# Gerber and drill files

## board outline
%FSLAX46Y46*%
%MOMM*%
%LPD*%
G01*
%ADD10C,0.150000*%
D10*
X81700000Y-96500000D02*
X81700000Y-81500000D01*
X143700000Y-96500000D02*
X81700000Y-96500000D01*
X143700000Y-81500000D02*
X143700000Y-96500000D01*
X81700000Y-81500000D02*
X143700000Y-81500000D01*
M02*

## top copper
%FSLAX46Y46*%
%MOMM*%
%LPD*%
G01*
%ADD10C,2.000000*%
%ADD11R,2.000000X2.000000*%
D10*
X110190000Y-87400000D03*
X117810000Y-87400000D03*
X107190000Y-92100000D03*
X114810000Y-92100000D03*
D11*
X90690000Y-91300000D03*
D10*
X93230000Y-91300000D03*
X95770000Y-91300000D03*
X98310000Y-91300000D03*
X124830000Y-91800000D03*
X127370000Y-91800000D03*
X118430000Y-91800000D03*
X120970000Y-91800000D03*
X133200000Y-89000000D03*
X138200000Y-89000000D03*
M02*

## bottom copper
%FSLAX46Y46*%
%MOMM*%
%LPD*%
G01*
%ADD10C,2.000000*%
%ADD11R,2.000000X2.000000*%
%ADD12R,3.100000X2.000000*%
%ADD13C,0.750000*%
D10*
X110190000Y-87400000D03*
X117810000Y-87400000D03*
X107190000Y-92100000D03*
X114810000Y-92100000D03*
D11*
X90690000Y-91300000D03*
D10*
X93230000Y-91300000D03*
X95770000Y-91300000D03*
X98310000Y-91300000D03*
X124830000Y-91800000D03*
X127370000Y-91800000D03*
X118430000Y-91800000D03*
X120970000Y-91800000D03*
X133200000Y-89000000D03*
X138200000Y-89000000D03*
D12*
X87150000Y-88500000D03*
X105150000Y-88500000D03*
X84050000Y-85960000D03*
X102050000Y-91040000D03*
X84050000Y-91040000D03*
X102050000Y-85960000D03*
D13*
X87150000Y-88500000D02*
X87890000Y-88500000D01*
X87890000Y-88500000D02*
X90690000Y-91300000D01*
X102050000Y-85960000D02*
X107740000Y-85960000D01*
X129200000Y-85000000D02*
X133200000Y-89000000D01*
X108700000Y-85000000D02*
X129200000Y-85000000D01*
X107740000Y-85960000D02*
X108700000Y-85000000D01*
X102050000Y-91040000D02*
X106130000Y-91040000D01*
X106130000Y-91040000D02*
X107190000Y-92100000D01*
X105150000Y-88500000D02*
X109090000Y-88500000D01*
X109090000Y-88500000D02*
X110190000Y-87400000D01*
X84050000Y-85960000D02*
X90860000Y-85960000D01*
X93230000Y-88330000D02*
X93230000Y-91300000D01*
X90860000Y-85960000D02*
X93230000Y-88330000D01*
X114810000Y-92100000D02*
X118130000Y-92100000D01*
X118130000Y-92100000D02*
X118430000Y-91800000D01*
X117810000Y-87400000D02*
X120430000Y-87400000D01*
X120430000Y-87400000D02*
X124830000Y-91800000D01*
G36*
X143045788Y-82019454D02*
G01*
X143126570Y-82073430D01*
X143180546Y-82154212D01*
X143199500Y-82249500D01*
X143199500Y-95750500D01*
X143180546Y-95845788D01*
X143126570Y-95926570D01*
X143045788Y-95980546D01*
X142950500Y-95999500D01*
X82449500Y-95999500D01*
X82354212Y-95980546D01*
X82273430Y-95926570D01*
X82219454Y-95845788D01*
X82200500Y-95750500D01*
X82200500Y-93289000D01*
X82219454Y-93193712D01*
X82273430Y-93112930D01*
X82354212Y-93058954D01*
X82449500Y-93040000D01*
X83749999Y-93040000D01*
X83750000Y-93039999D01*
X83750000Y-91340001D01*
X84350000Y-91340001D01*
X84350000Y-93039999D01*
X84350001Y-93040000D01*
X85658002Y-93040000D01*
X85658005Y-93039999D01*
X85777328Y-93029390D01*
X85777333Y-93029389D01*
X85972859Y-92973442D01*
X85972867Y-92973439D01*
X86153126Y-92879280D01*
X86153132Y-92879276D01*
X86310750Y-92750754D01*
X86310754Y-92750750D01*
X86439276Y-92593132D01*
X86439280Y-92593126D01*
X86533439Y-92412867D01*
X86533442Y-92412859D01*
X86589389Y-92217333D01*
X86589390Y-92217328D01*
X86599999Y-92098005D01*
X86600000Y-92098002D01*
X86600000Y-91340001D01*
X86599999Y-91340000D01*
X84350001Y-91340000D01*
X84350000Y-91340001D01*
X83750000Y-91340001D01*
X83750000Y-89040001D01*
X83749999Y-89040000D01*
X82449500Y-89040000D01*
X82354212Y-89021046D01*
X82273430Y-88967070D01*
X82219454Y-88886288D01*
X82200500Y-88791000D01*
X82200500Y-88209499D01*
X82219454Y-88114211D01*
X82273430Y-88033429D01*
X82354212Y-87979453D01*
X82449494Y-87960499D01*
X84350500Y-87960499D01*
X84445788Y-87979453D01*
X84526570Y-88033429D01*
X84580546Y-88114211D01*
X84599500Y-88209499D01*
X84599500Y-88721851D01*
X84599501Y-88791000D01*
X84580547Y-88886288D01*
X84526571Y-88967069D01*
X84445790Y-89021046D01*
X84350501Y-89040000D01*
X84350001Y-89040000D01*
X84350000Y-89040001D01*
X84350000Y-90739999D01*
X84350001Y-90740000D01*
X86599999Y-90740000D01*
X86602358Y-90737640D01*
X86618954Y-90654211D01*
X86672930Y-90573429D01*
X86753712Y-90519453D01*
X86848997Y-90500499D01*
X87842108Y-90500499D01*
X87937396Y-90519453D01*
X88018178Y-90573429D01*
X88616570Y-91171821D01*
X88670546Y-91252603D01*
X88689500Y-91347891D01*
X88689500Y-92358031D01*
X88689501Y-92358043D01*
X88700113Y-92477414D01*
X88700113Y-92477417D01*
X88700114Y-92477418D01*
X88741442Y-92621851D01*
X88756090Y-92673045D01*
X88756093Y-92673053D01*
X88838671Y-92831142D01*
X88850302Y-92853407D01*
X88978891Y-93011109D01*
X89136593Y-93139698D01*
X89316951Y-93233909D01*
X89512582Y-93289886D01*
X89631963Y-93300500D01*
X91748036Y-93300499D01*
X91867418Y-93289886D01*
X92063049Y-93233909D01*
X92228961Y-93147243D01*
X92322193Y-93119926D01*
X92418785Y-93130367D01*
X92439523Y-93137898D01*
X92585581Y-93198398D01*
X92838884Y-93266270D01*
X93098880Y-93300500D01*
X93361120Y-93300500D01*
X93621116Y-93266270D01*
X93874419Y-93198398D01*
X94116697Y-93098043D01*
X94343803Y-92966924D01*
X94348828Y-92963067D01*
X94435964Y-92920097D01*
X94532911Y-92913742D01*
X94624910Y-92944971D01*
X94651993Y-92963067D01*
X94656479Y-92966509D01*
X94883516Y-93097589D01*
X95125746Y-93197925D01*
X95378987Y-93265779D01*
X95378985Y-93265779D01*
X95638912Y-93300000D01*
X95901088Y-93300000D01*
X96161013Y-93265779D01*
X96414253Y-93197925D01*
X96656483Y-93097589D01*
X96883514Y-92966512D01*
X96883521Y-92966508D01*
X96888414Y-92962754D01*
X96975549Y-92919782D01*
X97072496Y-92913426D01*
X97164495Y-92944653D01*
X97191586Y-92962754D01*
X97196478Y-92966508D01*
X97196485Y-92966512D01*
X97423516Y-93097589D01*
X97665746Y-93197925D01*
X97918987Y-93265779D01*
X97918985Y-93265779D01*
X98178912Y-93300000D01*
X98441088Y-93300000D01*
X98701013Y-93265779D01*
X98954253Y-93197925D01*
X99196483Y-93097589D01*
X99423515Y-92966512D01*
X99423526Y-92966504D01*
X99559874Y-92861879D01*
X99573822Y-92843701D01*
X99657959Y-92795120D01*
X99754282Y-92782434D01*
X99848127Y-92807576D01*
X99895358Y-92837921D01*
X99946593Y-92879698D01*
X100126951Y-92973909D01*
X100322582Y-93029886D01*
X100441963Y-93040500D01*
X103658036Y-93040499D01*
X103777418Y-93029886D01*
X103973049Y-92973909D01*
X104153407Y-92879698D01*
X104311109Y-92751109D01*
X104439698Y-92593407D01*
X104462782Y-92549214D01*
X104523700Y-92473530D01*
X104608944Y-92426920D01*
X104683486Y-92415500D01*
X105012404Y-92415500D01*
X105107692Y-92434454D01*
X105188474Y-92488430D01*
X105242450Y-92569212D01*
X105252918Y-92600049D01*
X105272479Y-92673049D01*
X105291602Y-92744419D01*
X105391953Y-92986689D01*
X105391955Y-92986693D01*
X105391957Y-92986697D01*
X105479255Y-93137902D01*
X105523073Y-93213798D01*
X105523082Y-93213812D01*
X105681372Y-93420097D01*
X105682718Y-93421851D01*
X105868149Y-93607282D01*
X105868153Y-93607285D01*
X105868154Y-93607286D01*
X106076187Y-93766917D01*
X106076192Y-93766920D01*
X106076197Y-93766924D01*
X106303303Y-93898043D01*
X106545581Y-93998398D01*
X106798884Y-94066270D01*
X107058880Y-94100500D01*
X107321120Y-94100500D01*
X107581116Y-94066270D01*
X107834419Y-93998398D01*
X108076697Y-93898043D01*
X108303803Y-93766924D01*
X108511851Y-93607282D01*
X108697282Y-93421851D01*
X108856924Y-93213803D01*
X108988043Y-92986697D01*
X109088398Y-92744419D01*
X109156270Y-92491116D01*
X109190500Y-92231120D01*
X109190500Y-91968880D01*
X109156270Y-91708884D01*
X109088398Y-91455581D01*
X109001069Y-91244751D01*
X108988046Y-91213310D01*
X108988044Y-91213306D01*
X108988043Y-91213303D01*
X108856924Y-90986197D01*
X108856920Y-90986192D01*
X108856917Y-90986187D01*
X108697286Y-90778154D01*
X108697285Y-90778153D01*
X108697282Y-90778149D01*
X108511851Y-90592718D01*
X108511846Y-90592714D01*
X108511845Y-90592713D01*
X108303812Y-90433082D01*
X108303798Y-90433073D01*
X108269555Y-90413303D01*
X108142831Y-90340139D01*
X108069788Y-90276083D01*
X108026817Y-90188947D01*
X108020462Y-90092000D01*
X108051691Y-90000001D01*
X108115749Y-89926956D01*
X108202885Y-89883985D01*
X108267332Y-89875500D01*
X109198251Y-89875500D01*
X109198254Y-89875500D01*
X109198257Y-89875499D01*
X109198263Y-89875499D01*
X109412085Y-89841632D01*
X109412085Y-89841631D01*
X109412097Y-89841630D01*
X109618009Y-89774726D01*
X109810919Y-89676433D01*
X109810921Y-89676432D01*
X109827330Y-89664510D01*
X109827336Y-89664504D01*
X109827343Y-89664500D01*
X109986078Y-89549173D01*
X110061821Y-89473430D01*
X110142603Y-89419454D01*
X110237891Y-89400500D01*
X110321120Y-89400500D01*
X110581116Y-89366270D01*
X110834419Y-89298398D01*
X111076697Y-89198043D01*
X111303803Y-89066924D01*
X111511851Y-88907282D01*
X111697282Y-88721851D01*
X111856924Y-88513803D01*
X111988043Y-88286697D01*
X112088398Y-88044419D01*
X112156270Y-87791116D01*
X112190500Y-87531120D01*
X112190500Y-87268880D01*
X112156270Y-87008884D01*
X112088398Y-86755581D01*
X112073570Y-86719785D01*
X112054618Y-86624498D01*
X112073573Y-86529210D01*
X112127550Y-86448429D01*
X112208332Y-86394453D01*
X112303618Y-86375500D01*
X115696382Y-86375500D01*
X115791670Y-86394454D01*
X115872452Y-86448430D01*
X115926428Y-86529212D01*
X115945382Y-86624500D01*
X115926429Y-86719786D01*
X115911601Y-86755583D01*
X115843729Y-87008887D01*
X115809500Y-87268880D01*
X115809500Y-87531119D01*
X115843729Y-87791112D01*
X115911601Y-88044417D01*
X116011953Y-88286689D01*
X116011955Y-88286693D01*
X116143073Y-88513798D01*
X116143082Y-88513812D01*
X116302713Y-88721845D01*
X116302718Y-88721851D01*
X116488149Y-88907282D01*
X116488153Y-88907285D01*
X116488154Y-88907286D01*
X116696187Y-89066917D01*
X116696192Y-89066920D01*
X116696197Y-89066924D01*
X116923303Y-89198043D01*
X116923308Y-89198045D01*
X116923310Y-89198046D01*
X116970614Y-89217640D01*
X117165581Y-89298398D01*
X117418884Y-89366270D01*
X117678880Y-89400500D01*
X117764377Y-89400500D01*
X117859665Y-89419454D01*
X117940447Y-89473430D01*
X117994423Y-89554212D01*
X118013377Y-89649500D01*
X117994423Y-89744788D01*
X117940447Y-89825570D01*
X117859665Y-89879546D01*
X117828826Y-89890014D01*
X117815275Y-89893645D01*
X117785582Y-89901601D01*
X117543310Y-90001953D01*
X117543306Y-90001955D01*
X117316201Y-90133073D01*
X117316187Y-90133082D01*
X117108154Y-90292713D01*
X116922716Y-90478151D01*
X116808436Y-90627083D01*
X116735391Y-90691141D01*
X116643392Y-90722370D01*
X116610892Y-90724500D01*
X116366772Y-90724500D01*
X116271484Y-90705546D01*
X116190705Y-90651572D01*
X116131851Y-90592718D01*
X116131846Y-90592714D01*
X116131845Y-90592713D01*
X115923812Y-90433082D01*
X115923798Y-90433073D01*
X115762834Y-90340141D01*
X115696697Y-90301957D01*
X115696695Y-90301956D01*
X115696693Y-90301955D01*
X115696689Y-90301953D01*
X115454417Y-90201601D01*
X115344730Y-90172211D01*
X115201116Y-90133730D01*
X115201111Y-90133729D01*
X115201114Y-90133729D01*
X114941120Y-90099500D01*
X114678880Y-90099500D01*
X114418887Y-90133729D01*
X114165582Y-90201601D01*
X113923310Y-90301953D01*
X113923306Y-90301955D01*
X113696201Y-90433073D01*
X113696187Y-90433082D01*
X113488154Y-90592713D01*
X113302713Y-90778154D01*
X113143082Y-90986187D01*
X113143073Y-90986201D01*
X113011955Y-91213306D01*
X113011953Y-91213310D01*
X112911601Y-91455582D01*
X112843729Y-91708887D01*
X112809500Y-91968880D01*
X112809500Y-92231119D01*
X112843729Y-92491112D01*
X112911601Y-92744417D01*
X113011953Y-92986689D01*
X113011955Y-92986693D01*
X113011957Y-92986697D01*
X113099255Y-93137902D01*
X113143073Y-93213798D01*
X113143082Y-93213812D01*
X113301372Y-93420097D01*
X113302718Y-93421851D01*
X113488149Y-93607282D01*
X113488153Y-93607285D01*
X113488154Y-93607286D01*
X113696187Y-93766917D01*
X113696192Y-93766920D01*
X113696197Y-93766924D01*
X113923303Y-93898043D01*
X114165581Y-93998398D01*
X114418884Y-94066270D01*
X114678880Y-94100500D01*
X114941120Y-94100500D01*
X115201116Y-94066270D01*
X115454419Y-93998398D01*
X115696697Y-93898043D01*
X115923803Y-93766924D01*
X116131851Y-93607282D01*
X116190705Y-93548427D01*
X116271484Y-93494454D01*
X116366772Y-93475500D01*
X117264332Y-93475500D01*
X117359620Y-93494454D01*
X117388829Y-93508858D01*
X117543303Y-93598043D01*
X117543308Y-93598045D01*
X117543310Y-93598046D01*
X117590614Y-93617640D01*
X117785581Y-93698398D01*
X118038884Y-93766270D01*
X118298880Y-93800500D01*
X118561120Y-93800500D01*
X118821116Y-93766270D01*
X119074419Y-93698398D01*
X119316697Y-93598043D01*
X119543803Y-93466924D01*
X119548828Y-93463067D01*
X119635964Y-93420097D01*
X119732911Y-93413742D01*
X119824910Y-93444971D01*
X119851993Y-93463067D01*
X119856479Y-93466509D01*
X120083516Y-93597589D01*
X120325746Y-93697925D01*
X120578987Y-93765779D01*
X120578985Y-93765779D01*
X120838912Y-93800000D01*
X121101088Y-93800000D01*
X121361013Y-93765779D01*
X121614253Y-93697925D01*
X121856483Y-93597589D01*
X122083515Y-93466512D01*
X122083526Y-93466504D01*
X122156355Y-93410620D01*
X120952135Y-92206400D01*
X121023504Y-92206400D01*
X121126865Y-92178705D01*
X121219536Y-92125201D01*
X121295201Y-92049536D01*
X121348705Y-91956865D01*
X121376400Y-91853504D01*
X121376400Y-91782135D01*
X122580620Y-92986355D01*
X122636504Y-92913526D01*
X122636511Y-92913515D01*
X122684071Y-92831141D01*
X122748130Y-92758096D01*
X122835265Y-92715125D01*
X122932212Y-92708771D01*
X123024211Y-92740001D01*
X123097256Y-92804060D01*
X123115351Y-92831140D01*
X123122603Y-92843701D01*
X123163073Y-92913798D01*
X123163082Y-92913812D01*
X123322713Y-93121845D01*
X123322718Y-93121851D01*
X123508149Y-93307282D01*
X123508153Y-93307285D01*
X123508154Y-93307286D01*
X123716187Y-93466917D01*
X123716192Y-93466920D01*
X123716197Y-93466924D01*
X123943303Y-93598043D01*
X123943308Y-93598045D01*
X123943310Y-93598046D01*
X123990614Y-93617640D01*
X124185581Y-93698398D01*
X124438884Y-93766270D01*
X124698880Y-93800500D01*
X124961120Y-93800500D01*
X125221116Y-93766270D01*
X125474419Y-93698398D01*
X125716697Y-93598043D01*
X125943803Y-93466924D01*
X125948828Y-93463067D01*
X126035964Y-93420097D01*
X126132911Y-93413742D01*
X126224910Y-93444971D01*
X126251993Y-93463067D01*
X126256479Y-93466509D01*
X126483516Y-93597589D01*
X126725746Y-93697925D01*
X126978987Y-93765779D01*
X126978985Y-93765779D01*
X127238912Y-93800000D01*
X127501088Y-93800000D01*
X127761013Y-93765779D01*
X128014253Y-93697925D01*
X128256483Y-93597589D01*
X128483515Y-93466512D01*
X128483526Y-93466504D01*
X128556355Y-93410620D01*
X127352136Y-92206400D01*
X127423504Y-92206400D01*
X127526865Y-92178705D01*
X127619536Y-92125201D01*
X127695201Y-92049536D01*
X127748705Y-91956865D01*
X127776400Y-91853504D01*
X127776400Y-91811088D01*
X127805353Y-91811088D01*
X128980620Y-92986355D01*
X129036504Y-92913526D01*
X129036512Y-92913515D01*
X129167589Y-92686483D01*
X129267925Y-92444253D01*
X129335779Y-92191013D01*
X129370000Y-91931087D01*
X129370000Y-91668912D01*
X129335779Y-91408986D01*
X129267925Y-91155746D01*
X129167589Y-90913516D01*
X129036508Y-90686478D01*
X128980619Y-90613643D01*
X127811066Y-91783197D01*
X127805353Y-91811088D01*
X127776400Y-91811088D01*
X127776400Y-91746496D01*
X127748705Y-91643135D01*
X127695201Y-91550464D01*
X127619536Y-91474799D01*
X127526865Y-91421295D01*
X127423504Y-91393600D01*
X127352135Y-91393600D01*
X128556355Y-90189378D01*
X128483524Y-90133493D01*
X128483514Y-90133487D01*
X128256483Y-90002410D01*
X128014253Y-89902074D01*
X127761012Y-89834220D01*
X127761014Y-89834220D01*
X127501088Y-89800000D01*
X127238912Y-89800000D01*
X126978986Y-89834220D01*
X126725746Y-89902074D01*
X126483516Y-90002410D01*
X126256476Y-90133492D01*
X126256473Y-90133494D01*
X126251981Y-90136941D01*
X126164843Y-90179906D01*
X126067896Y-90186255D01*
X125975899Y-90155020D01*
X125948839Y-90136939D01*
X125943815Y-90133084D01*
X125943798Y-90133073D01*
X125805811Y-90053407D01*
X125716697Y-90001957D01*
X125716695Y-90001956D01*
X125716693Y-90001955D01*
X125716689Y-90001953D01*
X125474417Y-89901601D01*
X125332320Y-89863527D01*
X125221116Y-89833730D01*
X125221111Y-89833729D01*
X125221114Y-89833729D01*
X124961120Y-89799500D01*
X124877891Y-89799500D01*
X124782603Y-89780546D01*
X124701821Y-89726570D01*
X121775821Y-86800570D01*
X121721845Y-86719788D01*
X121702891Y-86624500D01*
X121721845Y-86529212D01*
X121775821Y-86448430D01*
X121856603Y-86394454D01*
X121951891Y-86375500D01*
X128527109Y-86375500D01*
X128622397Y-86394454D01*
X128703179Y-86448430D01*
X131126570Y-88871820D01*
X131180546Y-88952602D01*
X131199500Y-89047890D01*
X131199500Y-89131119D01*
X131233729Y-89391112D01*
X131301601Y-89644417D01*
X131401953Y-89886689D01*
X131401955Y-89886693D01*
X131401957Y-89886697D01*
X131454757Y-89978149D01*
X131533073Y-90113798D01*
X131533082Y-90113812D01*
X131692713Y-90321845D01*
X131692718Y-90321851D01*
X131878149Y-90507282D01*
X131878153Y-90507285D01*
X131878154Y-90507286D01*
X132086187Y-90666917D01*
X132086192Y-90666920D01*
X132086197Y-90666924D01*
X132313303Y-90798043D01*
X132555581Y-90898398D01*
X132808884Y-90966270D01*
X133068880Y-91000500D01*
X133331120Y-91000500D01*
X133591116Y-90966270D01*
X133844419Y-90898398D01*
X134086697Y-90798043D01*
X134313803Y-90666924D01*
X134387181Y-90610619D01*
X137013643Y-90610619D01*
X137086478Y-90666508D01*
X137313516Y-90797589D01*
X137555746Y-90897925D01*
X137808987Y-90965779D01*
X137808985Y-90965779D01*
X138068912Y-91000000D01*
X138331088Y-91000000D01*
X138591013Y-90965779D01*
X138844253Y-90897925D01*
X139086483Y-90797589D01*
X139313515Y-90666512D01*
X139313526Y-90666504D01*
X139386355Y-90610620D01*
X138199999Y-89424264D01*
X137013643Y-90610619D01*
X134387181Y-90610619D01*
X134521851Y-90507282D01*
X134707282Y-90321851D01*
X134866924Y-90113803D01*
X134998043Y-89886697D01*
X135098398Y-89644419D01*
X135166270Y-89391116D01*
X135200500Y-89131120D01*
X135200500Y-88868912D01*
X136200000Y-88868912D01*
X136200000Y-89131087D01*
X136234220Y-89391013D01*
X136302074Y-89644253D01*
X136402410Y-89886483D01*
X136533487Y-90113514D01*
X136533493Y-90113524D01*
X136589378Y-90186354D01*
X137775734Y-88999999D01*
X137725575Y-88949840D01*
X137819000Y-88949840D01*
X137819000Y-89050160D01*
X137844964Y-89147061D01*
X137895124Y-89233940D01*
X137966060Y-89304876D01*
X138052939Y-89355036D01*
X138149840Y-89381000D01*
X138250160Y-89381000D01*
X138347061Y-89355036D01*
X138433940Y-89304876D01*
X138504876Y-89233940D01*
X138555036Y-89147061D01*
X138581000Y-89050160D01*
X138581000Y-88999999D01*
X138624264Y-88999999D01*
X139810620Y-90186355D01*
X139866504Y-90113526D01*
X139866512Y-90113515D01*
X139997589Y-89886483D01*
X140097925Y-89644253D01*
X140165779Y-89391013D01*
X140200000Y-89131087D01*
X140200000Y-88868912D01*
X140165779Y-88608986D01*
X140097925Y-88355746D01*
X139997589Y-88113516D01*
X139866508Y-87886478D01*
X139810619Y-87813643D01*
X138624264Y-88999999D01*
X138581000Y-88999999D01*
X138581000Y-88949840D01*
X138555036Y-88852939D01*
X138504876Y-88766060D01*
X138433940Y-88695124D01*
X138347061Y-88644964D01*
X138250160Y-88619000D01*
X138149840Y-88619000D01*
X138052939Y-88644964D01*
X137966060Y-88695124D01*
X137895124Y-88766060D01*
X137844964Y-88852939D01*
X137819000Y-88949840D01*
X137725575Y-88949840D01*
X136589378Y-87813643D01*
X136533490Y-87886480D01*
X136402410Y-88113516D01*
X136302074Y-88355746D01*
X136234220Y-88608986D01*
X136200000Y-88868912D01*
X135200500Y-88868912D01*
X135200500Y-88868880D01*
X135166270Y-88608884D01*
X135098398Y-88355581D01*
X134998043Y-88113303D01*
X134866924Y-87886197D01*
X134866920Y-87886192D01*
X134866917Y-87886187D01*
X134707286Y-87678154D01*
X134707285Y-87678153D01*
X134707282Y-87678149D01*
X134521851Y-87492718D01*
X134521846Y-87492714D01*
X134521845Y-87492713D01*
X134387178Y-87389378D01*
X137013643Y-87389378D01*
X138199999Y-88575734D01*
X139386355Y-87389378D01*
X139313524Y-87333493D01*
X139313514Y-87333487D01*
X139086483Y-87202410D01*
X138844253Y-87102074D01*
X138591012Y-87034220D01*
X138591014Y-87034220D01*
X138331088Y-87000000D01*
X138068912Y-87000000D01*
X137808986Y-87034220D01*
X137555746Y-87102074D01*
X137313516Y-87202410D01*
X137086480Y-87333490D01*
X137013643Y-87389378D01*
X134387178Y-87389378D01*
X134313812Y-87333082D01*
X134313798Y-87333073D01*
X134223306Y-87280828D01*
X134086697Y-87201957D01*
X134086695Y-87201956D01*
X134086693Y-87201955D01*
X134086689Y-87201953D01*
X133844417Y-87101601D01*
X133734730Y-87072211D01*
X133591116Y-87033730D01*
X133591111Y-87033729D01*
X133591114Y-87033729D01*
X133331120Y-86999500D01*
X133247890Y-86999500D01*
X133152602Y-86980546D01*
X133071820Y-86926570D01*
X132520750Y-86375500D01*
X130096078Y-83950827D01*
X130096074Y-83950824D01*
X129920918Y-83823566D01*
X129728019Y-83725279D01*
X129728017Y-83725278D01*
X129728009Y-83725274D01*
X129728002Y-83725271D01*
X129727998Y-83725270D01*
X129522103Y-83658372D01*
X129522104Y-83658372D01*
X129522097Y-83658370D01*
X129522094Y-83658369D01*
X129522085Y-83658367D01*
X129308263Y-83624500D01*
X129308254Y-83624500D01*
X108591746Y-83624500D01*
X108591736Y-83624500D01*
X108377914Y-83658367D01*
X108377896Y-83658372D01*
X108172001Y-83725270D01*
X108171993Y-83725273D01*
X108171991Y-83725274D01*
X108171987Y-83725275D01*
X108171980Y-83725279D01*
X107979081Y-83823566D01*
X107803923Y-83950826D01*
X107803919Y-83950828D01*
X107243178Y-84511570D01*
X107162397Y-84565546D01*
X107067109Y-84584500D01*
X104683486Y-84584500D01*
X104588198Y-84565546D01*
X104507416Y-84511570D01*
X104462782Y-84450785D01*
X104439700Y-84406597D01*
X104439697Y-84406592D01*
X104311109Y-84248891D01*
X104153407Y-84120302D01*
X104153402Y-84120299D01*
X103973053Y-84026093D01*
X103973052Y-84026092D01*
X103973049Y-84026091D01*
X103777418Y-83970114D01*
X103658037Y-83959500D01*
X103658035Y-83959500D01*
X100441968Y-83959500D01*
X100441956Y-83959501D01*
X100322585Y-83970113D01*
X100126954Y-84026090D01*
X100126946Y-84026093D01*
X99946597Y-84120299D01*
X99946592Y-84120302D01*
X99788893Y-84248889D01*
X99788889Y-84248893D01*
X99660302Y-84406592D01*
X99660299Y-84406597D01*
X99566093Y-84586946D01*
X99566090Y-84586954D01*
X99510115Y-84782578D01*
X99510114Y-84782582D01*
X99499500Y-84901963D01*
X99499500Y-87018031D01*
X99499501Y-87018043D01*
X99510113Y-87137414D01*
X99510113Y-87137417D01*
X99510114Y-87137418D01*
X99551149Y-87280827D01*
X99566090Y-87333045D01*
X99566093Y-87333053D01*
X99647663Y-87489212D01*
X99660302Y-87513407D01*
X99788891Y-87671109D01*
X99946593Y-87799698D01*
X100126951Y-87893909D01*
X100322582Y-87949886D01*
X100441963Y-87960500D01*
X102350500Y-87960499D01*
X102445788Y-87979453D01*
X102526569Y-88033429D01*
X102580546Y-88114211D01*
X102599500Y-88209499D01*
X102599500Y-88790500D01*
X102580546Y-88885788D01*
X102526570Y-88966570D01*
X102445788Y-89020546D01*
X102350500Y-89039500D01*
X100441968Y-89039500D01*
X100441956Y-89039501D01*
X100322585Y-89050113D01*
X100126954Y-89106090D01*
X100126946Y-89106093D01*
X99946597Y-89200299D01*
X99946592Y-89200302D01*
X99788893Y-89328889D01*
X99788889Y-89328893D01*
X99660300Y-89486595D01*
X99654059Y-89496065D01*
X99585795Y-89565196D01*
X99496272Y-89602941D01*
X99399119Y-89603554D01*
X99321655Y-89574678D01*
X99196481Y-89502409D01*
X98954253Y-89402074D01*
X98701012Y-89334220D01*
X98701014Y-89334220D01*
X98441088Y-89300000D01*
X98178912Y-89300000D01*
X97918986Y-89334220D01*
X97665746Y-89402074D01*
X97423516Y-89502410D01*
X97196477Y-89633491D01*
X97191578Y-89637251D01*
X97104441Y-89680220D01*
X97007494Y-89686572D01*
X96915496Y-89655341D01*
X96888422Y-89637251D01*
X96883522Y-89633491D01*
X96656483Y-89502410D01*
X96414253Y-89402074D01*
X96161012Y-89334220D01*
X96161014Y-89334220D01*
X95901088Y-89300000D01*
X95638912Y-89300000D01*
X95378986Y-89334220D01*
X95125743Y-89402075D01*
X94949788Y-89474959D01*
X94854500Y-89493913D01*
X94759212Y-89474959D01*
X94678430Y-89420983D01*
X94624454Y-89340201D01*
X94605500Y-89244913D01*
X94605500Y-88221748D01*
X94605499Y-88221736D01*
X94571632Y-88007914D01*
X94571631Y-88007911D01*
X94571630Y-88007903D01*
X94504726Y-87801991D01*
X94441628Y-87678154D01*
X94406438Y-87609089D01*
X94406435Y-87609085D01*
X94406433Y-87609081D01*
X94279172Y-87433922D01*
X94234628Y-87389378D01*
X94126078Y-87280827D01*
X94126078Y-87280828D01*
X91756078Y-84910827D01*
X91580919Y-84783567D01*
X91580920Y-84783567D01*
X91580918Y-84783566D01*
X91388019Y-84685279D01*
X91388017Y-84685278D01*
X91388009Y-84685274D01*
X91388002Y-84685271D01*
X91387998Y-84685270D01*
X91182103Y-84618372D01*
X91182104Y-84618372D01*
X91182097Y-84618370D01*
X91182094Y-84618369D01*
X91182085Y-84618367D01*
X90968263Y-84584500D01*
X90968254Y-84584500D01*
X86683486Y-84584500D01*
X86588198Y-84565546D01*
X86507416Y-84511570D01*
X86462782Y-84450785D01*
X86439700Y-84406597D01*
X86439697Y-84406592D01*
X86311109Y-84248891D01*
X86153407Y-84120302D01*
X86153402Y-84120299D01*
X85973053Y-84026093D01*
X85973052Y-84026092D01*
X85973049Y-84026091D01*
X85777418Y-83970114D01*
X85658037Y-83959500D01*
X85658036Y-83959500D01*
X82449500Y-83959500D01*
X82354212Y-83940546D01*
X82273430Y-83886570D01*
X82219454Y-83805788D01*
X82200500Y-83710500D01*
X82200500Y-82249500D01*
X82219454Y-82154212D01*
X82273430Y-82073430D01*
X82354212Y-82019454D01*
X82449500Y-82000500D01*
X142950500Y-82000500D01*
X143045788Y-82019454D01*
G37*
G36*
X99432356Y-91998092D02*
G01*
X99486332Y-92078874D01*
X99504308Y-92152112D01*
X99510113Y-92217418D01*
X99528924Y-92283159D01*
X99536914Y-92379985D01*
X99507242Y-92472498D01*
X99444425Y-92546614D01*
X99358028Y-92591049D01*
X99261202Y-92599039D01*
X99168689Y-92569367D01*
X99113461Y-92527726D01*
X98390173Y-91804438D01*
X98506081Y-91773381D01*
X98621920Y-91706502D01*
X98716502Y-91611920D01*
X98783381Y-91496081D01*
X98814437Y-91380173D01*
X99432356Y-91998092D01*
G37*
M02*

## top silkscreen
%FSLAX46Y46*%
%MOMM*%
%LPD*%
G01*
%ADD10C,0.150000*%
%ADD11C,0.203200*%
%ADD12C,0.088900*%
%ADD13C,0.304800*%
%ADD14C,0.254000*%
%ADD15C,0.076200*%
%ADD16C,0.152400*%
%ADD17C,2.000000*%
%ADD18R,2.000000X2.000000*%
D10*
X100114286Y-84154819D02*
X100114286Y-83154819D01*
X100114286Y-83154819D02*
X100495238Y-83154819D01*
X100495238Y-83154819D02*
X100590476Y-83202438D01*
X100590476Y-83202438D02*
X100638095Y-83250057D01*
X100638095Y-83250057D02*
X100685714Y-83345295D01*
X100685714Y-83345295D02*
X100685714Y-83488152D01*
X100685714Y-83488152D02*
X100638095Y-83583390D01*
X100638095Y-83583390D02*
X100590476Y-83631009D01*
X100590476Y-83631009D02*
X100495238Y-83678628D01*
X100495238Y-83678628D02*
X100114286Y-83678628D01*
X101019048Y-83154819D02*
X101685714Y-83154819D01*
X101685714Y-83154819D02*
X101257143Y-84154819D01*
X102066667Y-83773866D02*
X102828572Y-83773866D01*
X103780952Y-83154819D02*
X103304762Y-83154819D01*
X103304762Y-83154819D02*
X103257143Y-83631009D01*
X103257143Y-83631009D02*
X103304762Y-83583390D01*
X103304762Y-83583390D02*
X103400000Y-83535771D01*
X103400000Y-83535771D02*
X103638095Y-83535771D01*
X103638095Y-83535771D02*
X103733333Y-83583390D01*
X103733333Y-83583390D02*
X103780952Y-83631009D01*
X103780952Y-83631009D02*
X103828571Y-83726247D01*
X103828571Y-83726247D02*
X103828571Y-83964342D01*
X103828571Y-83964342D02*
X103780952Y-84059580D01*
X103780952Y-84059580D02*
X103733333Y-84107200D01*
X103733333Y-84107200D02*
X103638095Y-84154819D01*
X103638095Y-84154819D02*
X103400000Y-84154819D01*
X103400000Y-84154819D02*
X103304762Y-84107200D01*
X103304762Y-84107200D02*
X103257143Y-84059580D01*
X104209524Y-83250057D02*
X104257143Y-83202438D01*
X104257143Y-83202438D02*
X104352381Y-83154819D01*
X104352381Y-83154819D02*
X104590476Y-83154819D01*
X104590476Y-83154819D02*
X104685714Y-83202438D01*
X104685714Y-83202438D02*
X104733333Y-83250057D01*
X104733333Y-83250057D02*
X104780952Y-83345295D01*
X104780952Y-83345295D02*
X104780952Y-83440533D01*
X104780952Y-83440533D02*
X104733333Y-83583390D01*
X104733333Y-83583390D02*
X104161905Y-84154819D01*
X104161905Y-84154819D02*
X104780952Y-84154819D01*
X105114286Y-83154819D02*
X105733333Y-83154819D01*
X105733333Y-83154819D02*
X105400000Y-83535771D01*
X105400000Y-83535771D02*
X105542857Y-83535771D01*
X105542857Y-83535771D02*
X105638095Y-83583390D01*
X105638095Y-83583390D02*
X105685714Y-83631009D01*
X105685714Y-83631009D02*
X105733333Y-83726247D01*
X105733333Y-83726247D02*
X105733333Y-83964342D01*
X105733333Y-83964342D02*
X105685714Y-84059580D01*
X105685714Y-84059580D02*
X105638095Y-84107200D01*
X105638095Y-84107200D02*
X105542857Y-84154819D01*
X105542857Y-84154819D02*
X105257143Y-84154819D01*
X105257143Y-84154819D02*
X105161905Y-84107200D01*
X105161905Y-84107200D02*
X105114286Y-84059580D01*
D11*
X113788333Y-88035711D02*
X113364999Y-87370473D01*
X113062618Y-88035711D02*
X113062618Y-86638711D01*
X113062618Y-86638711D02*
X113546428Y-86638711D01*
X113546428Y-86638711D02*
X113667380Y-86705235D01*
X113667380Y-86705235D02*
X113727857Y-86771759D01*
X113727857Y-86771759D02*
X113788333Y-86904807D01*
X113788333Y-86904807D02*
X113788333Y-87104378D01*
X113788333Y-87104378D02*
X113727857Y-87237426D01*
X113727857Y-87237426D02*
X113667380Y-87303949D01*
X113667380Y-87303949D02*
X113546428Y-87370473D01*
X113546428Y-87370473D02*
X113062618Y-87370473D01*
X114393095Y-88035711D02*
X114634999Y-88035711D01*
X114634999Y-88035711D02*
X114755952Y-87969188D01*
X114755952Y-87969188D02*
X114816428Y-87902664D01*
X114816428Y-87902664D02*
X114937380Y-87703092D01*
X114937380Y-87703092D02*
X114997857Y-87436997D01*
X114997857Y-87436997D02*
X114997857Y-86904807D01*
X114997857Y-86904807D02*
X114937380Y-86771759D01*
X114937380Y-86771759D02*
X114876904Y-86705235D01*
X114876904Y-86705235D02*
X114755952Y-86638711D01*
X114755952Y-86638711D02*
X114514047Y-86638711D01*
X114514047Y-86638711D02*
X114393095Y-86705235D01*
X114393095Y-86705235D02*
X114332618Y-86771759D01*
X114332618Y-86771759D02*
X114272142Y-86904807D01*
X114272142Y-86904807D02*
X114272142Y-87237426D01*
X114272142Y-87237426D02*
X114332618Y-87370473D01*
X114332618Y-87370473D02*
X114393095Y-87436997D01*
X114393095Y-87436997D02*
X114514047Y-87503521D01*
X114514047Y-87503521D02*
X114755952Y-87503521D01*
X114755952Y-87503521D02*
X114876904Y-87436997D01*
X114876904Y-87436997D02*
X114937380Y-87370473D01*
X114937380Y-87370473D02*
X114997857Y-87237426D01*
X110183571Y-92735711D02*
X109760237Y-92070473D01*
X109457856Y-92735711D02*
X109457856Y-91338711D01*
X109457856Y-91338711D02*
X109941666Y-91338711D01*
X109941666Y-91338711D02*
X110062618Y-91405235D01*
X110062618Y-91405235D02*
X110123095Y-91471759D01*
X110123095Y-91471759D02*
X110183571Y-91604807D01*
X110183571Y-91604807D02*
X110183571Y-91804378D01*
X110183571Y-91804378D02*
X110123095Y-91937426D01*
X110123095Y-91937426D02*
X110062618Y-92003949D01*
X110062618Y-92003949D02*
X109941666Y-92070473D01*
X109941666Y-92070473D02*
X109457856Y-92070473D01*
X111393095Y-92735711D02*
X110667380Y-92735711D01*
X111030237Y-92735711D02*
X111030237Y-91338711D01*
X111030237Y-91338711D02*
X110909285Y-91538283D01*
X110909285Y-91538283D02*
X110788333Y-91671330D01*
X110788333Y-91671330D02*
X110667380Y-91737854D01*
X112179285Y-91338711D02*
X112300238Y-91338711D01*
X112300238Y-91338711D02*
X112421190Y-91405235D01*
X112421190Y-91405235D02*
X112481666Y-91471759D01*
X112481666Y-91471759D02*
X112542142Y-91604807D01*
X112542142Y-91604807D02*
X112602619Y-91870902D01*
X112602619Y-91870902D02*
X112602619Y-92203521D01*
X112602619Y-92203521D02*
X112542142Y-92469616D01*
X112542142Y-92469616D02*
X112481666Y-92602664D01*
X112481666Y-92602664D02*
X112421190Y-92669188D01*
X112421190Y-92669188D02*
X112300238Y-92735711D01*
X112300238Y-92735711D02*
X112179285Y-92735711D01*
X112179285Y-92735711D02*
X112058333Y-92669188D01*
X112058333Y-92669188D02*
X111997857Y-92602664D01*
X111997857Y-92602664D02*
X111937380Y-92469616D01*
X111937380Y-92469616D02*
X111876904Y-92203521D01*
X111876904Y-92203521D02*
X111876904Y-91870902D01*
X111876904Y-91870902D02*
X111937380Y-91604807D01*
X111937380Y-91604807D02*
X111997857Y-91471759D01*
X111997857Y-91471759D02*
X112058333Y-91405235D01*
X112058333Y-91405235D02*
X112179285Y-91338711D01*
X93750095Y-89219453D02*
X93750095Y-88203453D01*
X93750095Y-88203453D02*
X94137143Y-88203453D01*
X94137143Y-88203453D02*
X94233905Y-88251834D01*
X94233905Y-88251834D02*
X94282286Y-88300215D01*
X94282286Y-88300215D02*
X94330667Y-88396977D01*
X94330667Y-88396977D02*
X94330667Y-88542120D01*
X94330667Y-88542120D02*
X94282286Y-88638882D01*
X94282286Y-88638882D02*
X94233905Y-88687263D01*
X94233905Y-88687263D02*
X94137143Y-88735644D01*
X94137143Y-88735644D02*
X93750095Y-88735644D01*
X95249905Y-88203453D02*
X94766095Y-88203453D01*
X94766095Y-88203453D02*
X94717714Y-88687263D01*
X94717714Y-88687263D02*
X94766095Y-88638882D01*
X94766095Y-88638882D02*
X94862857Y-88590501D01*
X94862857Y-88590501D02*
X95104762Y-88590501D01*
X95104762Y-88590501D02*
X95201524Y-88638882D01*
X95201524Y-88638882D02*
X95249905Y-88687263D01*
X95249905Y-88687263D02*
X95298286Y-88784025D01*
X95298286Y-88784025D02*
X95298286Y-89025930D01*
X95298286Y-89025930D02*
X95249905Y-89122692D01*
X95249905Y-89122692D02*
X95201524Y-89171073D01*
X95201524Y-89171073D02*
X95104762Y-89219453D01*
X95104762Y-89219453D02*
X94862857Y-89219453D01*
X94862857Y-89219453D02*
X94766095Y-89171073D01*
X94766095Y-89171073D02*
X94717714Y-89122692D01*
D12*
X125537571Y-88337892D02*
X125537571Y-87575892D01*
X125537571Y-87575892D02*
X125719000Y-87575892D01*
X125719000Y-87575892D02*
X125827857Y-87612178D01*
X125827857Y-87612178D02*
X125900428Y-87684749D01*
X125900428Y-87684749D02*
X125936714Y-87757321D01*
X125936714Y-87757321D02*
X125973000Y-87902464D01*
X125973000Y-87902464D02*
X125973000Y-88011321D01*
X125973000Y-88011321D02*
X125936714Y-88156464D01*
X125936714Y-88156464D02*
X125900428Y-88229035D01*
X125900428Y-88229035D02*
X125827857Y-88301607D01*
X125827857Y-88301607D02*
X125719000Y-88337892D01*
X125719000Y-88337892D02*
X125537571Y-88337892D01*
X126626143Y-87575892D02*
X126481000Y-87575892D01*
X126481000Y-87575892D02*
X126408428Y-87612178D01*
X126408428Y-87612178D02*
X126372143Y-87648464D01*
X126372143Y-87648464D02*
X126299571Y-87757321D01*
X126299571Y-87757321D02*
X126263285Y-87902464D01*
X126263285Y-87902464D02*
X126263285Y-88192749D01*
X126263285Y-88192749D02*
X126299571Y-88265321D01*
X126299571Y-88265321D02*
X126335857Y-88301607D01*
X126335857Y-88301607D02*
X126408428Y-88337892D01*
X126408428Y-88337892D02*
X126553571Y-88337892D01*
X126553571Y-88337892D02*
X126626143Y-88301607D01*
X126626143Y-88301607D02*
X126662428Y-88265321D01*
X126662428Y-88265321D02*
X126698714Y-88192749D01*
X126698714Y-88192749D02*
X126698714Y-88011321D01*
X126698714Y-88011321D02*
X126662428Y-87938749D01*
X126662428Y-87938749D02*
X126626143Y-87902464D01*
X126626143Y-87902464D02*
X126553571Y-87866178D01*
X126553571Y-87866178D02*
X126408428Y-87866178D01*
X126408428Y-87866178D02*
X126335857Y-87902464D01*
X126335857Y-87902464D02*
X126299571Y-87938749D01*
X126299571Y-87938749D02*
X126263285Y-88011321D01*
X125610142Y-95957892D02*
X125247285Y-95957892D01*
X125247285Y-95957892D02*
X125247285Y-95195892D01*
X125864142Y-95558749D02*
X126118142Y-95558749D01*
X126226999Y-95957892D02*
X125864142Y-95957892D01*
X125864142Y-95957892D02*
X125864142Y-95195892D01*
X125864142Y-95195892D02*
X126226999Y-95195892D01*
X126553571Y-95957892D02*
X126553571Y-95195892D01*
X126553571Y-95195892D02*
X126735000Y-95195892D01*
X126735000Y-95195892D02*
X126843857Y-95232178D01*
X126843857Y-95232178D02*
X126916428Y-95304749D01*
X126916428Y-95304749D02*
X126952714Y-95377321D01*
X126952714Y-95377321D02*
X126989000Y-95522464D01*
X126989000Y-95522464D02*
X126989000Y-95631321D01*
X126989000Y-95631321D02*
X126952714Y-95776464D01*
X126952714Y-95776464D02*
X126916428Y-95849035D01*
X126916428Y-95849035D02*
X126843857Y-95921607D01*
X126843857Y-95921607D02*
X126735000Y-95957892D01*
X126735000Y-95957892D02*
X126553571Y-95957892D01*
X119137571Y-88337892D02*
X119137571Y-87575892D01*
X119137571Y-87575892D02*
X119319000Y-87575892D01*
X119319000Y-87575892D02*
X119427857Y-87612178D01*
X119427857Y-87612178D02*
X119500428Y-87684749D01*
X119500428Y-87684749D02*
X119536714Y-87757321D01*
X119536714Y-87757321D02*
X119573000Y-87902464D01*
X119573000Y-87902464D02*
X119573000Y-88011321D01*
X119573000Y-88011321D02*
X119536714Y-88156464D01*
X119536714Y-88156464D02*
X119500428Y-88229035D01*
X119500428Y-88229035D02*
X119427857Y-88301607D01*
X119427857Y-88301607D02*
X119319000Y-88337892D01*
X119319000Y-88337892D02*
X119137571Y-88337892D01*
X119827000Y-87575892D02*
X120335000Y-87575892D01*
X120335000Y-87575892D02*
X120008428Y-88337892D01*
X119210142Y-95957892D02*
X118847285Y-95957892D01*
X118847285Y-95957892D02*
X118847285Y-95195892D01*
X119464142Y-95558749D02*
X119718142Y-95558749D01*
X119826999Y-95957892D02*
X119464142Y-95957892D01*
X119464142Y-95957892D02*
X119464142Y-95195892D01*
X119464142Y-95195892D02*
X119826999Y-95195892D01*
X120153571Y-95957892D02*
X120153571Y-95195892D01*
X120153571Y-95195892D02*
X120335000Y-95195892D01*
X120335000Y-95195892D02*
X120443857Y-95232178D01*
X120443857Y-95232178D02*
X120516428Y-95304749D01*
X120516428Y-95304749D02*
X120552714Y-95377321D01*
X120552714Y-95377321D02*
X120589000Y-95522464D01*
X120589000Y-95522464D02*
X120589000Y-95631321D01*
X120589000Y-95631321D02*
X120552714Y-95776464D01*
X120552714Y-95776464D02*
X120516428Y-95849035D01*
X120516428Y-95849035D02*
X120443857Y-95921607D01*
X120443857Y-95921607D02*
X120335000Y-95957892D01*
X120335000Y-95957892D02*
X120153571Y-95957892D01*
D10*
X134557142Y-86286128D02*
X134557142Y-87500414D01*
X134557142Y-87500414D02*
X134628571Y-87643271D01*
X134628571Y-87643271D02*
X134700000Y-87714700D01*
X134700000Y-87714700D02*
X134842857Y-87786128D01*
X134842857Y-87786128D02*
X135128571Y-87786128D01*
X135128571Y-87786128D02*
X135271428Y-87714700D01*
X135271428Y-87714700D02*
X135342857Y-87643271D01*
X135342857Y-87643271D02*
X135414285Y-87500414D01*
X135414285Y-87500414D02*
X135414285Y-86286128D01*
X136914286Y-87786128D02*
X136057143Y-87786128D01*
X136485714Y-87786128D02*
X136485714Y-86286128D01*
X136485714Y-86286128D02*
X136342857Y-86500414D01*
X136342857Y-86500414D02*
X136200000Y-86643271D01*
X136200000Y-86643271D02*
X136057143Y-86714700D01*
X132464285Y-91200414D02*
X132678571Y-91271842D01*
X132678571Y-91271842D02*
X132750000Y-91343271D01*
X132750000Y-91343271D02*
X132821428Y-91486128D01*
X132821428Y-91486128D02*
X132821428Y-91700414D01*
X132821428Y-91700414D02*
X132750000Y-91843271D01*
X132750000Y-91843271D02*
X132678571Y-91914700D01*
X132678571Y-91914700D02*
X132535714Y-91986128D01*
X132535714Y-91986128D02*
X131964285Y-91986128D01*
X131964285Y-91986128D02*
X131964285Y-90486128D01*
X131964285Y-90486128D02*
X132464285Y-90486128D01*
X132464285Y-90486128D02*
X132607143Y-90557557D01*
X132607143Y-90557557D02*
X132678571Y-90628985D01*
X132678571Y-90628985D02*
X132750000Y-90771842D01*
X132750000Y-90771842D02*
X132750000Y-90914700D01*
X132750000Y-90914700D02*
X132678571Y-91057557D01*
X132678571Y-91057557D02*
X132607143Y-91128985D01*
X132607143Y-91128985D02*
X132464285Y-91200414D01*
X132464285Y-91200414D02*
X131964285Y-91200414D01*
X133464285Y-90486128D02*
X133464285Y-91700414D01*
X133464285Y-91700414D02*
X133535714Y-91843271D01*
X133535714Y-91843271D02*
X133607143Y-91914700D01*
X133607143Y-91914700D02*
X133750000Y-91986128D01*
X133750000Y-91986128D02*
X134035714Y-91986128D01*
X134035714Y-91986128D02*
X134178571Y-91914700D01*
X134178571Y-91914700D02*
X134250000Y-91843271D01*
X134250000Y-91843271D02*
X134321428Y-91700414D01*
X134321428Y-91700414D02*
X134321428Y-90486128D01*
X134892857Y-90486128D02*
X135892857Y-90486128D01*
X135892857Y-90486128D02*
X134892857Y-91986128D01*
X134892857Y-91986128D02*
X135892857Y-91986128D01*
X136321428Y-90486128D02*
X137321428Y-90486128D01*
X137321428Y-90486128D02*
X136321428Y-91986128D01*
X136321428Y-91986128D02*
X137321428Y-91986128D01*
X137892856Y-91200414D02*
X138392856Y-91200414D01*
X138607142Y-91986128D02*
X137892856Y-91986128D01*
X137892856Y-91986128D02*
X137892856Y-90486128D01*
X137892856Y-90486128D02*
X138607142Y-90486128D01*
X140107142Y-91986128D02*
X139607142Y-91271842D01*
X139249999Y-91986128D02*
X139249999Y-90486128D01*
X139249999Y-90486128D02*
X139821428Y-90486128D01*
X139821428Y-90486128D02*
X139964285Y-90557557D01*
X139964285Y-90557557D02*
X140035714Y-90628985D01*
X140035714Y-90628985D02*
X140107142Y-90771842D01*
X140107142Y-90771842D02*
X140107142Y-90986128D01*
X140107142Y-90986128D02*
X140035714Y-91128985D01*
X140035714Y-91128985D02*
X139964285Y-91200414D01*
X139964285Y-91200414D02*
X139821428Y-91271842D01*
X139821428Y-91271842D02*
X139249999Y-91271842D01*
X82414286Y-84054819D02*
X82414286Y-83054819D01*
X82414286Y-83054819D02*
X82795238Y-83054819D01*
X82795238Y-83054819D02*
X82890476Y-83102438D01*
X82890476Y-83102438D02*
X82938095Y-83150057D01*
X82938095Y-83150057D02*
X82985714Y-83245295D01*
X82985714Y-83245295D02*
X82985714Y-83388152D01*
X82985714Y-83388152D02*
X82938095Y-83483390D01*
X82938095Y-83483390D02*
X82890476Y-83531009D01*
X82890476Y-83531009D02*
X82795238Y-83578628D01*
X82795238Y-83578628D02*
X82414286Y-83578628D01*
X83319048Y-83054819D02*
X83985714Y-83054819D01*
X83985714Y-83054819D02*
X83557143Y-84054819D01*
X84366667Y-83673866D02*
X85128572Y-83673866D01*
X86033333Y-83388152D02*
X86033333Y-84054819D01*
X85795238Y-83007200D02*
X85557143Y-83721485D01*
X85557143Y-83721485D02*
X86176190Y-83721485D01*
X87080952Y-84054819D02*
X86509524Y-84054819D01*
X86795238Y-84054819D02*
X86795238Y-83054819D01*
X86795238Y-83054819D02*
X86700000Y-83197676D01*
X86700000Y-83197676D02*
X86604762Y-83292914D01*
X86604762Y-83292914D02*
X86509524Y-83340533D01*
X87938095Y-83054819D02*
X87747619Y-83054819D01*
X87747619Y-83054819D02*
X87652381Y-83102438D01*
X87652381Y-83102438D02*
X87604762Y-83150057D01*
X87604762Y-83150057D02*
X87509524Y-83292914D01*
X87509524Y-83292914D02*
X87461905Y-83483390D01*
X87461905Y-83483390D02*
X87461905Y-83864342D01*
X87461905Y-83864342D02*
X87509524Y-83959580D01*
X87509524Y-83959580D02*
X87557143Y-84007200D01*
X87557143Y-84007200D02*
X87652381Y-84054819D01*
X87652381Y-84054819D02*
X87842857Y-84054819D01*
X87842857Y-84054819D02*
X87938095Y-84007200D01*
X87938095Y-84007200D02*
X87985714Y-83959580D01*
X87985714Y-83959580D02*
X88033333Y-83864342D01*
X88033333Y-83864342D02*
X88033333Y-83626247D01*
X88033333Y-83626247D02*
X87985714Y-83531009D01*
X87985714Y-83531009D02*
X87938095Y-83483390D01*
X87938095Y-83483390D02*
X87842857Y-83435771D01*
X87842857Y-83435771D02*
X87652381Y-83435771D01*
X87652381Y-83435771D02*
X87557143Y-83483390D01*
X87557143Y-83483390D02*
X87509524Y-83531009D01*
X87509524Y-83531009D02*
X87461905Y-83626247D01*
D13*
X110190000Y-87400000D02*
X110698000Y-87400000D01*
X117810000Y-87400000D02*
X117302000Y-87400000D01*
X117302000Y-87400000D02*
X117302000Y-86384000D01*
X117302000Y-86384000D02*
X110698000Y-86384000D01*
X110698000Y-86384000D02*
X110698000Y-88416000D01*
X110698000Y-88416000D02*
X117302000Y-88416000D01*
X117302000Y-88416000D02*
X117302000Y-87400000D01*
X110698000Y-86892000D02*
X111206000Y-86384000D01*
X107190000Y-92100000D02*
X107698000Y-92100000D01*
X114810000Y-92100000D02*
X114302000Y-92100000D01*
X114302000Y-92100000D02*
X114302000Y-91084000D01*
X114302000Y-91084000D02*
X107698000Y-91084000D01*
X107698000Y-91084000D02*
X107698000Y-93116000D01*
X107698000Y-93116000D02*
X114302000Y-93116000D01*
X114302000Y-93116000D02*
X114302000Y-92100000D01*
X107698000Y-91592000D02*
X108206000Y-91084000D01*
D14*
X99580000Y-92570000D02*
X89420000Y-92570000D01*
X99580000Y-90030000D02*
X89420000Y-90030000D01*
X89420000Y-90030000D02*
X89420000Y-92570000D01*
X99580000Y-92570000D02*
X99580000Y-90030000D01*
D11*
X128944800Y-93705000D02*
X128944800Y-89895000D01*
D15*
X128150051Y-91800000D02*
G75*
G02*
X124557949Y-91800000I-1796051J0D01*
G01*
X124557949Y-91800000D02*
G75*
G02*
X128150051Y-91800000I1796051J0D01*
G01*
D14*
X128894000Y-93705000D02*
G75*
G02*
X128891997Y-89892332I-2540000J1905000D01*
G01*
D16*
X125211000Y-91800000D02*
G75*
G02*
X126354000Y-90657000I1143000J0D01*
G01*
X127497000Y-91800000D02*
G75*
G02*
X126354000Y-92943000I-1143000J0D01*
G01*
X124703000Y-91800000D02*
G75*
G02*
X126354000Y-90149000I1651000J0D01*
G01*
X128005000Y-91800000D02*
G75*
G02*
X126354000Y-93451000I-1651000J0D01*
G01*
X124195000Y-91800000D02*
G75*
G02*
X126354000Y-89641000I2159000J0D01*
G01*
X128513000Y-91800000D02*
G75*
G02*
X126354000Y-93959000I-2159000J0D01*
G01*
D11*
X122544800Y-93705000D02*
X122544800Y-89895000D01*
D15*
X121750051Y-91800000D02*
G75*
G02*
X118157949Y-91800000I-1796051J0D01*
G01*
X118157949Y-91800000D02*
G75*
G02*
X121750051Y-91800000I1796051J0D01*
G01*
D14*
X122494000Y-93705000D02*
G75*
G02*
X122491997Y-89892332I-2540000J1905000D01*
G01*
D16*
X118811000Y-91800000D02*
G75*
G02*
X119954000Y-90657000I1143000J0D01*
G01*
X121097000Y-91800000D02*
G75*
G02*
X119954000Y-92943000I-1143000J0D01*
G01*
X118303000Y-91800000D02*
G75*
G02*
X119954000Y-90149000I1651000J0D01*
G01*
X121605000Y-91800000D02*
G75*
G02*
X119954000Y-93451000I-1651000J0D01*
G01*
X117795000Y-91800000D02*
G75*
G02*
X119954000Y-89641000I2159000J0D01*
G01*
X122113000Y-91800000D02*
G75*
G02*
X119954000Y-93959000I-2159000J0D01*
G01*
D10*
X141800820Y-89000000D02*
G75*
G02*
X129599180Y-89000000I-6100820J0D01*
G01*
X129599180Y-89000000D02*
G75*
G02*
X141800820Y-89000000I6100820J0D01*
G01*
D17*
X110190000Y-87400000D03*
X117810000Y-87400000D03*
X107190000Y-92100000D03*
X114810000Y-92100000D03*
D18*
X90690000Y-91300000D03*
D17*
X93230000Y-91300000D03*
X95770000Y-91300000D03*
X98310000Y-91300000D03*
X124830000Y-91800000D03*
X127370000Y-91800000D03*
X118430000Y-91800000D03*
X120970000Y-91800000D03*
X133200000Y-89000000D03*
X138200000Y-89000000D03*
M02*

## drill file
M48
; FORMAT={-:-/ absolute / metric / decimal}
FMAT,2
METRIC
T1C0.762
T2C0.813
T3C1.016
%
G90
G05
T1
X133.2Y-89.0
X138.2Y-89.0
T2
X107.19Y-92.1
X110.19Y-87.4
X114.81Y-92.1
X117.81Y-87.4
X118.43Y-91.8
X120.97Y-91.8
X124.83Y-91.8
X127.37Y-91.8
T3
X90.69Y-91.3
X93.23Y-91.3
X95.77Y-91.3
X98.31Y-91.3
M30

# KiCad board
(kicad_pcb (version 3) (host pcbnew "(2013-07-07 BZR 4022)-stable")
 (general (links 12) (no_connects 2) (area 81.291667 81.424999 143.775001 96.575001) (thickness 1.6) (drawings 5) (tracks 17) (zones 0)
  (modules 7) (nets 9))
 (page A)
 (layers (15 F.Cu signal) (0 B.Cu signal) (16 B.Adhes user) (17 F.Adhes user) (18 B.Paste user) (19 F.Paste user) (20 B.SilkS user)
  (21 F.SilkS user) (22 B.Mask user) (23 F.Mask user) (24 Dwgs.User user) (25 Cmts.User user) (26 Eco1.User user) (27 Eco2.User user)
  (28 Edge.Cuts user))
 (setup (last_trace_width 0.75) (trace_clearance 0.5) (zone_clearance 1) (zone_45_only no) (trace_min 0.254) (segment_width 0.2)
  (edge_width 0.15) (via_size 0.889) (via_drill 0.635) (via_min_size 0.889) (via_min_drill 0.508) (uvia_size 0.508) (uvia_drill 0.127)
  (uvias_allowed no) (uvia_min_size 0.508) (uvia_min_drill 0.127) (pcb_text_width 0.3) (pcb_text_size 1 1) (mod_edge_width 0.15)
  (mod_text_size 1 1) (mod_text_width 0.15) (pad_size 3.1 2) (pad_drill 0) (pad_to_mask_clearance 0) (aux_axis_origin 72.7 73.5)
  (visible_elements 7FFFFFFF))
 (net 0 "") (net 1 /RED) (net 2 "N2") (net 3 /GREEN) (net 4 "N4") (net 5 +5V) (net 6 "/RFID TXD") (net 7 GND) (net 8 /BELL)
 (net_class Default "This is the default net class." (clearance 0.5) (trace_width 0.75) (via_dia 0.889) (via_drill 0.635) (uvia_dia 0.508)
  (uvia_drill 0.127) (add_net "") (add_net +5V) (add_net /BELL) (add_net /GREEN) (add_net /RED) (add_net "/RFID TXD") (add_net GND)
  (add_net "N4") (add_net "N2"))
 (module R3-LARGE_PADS (layer F.Cu) (at 114 87.4) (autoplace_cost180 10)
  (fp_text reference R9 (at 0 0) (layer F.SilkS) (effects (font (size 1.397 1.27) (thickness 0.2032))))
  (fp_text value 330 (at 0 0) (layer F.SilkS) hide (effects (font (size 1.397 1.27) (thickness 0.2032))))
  (fp_line (start -3.81 0) (end -3.302 0) (layer F.SilkS) (width 0.3048))
  (fp_line (start 3.81 0) (end 3.302 0) (layer F.SilkS) (width 0.3048))
  (fp_line (start 3.302 0) (end 3.302 -1.016) (layer F.SilkS) (width 0.3048))
  (fp_line (start 3.302 -1.016) (end -3.302 -1.016) (layer F.SilkS) (width 0.3048))
  (fp_line (start -3.302 -1.016) (end -3.302 1.016) (layer F.SilkS) (width 0.3048))
  (fp_line (start -3.302 1.016) (end 3.302 1.016) (layer F.SilkS) (width 0.3048))
  (fp_line (start 3.302 1.016) (end 3.302 0) (layer F.SilkS) (width 0.3048))
  (fp_line (start -3.302 -0.508) (end -2.794 -1.016) (layer F.SilkS) (width 0.3048))
  (pad 1 thru_hole circle (at -3.81 0) (size 2 2) (drill 0.8128) (layers *.Cu *.Mask F.SilkS) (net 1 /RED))
  (pad 2 thru_hole circle (at 3.81 0) (size 2 2) (drill 0.8128) (layers *.Cu *.Mask F.SilkS) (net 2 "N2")))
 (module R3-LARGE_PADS (layer F.Cu) (at 111 92.1) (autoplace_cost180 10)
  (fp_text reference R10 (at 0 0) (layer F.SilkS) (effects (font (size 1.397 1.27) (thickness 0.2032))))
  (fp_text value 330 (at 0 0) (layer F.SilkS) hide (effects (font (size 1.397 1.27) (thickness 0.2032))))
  (fp_line (start -3.81 0) (end -3.302 0) (layer F.SilkS) (width 0.3048))
  (fp_line (start 3.81 0) (end 3.302 0) (layer F.SilkS) (width 0.3048))
  (fp_line (start 3.302 0) (end 3.302 -1.016) (layer F.SilkS) (width 0.3048))
  (fp_line (start 3.302 -1.016) (end -3.302 -1.016) (layer F.SilkS) (width 0.3048))
  (fp_line (start -3.302 -1.016) (end -3.302 1.016) (layer F.SilkS) (width 0.3048))
  (fp_line (start -3.302 1.016) (end 3.302 1.016) (layer F.SilkS) (width 0.3048))
  (fp_line (start 3.302 1.016) (end 3.302 0) (layer F.SilkS) (width 0.3048))
  (fp_line (start -3.302 -0.508) (end -2.794 -1.016) (layer F.SilkS) (width 0.3048))
  (pad 1 thru_hole circle (at -3.81 0) (size 2 2) (drill 0.8128) (layers *.Cu *.Mask F.SilkS) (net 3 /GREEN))
  (pad 2 thru_hole circle (at 3.81 0) (size 2 2) (drill 0.8128) (layers *.Cu *.Mask F.SilkS) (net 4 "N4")))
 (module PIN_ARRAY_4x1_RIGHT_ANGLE (layer F.Cu) (at 94.5 91.3)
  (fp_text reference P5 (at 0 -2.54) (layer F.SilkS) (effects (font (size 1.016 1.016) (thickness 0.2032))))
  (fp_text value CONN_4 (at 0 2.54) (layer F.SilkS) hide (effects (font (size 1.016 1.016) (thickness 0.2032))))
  (fp_line (start 5.08 1.27) (end -5.08 1.27) (layer F.SilkS) (width 0.254))
  (fp_line (start 5.08 -1.27) (end -5.08 -1.27) (layer F.SilkS) (width 0.254))
  (fp_line (start -5.08 -1.27) (end -5.08 1.27) (layer F.SilkS) (width 0.254))
  (fp_line (start 5.08 1.27) (end 5.08 -1.27) (layer F.SilkS) (width 0.254))
  (pad 1 thru_hole rect (at -3.81 0) (size 2 2) (drill 1.016) (layers *.Cu *.Mask F.SilkS) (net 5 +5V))
  (pad 2 thru_hole circle (at -1.27 0) (size 2 2) (drill 1.016) (layers *.Cu *.Mask F.SilkS) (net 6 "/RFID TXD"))
  (pad 3 thru_hole circle (at 1.27 0) (size 2 2) (drill 1.016) (layers *.Cu *.Mask F.SilkS) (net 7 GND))
  (pad 4 thru_hole circle (at 3.81 0) (size 2 2) (drill 1.016) (layers *.Cu *.Mask F.SilkS) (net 7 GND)))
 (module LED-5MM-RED (layer F.Cu) (at 126.1 91.8)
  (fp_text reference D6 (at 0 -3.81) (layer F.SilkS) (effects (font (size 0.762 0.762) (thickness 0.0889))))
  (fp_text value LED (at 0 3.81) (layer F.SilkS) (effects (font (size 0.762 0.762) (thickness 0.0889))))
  (fp_line (start 2.8448 1.905) (end 2.8448 -1.905) (layer F.SilkS) (width 0.2032))
  (fp_circle (center 0.254 0) (end -1.016 1.27) (layer F.SilkS) (width 0.0762))
  (fp_arc (start 0.254 0) (end 2.794 1.905) (angle 286.2) (layer F.SilkS) (width 0.254))
  (fp_arc (start 0.254 0) (end -0.889 0) (angle 90) (layer F.SilkS) (width 0.1524))
  (fp_arc (start 0.254 0) (end 1.397 0) (angle 90) (layer F.SilkS) (width 0.1524))
  (fp_arc (start 0.254 0) (end -1.397 0) (angle 90) (layer F.SilkS) (width 0.1524))
  (fp_arc (start 0.254 0) (end 1.905 0) (angle 90) (layer F.SilkS) (width 0.1524))
  (fp_arc (start 0.254 0) (end -1.905 0) (angle 90) (layer F.SilkS) (width 0.1524))
  (fp_arc (start 0.254 0) (end 2.413 0) (angle 90) (layer F.SilkS) (width 0.1524))
  (pad 1 thru_hole circle (at -1.27 0) (size 2 2) (drill 0.8128) (layers *.Cu *.Mask F.SilkS) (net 2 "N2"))
  (pad 2 thru_hole circle (at 1.27 0) (size 2 2) (drill 0.8128) (layers *.Cu *.Mask F.SilkS) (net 7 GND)))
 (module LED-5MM (layer F.Cu) (at 119.7 91.8)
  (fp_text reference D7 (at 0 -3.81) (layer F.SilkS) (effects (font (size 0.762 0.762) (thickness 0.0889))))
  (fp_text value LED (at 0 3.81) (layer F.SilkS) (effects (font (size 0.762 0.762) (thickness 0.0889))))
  (fp_line (start 2.8448 1.905) (end 2.8448 -1.905) (layer F.SilkS) (width 0.2032))
  (fp_circle (center 0.254 0) (end -1.016 1.27) (layer F.SilkS) (width 0.0762))
  (fp_arc (start 0.254 0) (end 2.794 1.905) (angle 286.2) (layer F.SilkS) (width 0.254))
  (fp_arc (start 0.254 0) (end -0.889 0) (angle 90) (layer F.SilkS) (width 0.1524))
  (fp_arc (start 0.254 0) (end 1.397 0) (angle 90) (layer F.SilkS) (width 0.1524))
  (fp_arc (start 0.254 0) (end -1.397 0) (angle 90) (layer F.SilkS) (width 0.1524))
  (fp_arc (start 0.254 0) (end 1.905 0) (angle 90) (layer F.SilkS) (width 0.1524))
  (fp_arc (start 0.254 0) (end -1.905 0) (angle 90) (layer F.SilkS) (width 0.1524))
  (fp_arc (start 0.254 0) (end 2.413 0) (angle 90) (layer F.SilkS) (width 0.1524))
  (pad 1 thru_hole circle (at -1.27 0) (size 2 2) (drill 0.8128) (layers *.Cu *.Mask F.SilkS) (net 4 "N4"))
  (pad 2 thru_hole circle (at 1.27 0) (size 2 2) (drill 0.8128) (layers *.Cu *.Mask F.SilkS) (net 7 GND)))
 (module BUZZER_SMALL (layer F.Cu) (at 135.7 89)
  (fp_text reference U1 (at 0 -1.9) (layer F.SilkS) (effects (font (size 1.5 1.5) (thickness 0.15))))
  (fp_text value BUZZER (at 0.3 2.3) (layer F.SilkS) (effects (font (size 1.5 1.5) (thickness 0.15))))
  (fp_circle (center 0 0) (end 6.1 0.1) (layer F.SilkS) (width 0.15))
  (pad 1 thru_hole circle (at -2.5 0) (size 2 2) (drill 0.762) (layers *.Cu *.Mask F.SilkS) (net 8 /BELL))
  (pad 2 thru_hole circle (at 2.5 0) (size 2 2) (drill 0.762) (layers *.Cu *.Mask F.SilkS) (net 7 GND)))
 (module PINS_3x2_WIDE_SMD (layer F.Cu) (at 94.6 88.5)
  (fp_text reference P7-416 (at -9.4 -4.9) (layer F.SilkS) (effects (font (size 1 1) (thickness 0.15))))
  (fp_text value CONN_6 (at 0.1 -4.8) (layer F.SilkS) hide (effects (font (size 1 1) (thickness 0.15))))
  (pad 1 smd rect (at -7.45 0) (size 3.1 2) (layers B.Cu B.Paste B.SilkS B.Mask) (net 5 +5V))
  (pad 2 smd rect (at 10.55 0) (size 3.1 2) (layers B.Cu B.Paste B.SilkS B.Mask) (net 1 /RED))
  (pad 4 smd rect (at -10.55 -2.54) (size 3.1 2) (layers B.Cu B.Paste B.SilkS B.Mask) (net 6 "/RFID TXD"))
  (pad 3 smd rect (at 7.45 2.54) (size 3.1 2) (layers B.Cu B.Paste B.SilkS B.Mask) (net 3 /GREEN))
  (pad 6 smd rect (at -10.55 2.54) (size 3.1 2) (layers B.Cu B.Paste B.SilkS B.Mask) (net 7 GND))
  (pad 5 smd rect (at 7.45 -2.54) (size 3.1 2) (layers B.Cu B.Paste B.SilkS B.Mask) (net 8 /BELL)))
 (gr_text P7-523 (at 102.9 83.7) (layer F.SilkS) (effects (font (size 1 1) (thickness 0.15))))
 (gr_line (start 81.7 96.5) (end 81.7 81.5) (angle 90) (layer Edge.Cuts) (width 0.15))
 (gr_line (start 143.7 96.5) (end 81.7 96.5) (angle 90) (layer Edge.Cuts) (width 0.15))
 (gr_line (start 143.7 81.5) (end 143.7 96.5) (angle 90) (layer Edge.Cuts) (width 0.15))
 (gr_line (start 81.7 81.5) (end 143.7 81.5) (angle 90) (layer Edge.Cuts) (width 0.15))
 (segment (start 87.15 88.5) (end 87.89 88.5) (width 0.75) (layer B.Cu) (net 5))
 (segment (start 87.89 88.5) (end 90.69 91.3) (width 0.75) (layer B.Cu) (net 5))
 (segment (start 102.05 85.96) (end 107.74 85.96) (width 0.75) (layer B.Cu) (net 8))
 (segment (start 129.2 85) (end 133.2 89) (width 0.75) (layer B.Cu) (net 8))
 (segment (start 108.7 85) (end 129.2 85) (width 0.75) (layer B.Cu) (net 8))
 (segment (start 107.74 85.96) (end 108.7 85) (width 0.75) (layer B.Cu) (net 8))
 (segment (start 102.05 91.04) (end 106.13 91.04) (width 0.75) (layer B.Cu) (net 3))
 (segment (start 106.13 91.04) (end 107.19 92.1) (width 0.75) (layer B.Cu) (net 3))
 (segment (start 105.15 88.5) (end 109.09 88.5) (width 0.75) (layer B.Cu) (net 1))
 (segment (start 109.09 88.5) (end 110.19 87.4) (width 0.75) (layer B.Cu) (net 1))
 (segment (start 84.05 85.96) (end 90.86 85.96) (width 0.75) (layer B.Cu) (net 6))
 (segment (start 93.23 88.33) (end 93.23 91.3) (width 0.75) (layer B.Cu) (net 6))
 (segment (start 90.86 85.96) (end 93.23 88.33) (width 0.75) (layer B.Cu) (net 6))
 (segment (start 114.81 92.1) (end 118.13 92.1) (width 0.75) (layer B.Cu) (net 4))
 (segment (start 118.13 92.1) (end 118.43 91.8) (width 0.75) (layer B.Cu) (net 4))
 (segment (start 117.81 87.4) (end 120.43 87.4) (width 0.75) (layer B.Cu) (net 2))
 (segment (start 120.43 87.4) (end 124.83 91.8) (width 0.75) (layer B.Cu) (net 2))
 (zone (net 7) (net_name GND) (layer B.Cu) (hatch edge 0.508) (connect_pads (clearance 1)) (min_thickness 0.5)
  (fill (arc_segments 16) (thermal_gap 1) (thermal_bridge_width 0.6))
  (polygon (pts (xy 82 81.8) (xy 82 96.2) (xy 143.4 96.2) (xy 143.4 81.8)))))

